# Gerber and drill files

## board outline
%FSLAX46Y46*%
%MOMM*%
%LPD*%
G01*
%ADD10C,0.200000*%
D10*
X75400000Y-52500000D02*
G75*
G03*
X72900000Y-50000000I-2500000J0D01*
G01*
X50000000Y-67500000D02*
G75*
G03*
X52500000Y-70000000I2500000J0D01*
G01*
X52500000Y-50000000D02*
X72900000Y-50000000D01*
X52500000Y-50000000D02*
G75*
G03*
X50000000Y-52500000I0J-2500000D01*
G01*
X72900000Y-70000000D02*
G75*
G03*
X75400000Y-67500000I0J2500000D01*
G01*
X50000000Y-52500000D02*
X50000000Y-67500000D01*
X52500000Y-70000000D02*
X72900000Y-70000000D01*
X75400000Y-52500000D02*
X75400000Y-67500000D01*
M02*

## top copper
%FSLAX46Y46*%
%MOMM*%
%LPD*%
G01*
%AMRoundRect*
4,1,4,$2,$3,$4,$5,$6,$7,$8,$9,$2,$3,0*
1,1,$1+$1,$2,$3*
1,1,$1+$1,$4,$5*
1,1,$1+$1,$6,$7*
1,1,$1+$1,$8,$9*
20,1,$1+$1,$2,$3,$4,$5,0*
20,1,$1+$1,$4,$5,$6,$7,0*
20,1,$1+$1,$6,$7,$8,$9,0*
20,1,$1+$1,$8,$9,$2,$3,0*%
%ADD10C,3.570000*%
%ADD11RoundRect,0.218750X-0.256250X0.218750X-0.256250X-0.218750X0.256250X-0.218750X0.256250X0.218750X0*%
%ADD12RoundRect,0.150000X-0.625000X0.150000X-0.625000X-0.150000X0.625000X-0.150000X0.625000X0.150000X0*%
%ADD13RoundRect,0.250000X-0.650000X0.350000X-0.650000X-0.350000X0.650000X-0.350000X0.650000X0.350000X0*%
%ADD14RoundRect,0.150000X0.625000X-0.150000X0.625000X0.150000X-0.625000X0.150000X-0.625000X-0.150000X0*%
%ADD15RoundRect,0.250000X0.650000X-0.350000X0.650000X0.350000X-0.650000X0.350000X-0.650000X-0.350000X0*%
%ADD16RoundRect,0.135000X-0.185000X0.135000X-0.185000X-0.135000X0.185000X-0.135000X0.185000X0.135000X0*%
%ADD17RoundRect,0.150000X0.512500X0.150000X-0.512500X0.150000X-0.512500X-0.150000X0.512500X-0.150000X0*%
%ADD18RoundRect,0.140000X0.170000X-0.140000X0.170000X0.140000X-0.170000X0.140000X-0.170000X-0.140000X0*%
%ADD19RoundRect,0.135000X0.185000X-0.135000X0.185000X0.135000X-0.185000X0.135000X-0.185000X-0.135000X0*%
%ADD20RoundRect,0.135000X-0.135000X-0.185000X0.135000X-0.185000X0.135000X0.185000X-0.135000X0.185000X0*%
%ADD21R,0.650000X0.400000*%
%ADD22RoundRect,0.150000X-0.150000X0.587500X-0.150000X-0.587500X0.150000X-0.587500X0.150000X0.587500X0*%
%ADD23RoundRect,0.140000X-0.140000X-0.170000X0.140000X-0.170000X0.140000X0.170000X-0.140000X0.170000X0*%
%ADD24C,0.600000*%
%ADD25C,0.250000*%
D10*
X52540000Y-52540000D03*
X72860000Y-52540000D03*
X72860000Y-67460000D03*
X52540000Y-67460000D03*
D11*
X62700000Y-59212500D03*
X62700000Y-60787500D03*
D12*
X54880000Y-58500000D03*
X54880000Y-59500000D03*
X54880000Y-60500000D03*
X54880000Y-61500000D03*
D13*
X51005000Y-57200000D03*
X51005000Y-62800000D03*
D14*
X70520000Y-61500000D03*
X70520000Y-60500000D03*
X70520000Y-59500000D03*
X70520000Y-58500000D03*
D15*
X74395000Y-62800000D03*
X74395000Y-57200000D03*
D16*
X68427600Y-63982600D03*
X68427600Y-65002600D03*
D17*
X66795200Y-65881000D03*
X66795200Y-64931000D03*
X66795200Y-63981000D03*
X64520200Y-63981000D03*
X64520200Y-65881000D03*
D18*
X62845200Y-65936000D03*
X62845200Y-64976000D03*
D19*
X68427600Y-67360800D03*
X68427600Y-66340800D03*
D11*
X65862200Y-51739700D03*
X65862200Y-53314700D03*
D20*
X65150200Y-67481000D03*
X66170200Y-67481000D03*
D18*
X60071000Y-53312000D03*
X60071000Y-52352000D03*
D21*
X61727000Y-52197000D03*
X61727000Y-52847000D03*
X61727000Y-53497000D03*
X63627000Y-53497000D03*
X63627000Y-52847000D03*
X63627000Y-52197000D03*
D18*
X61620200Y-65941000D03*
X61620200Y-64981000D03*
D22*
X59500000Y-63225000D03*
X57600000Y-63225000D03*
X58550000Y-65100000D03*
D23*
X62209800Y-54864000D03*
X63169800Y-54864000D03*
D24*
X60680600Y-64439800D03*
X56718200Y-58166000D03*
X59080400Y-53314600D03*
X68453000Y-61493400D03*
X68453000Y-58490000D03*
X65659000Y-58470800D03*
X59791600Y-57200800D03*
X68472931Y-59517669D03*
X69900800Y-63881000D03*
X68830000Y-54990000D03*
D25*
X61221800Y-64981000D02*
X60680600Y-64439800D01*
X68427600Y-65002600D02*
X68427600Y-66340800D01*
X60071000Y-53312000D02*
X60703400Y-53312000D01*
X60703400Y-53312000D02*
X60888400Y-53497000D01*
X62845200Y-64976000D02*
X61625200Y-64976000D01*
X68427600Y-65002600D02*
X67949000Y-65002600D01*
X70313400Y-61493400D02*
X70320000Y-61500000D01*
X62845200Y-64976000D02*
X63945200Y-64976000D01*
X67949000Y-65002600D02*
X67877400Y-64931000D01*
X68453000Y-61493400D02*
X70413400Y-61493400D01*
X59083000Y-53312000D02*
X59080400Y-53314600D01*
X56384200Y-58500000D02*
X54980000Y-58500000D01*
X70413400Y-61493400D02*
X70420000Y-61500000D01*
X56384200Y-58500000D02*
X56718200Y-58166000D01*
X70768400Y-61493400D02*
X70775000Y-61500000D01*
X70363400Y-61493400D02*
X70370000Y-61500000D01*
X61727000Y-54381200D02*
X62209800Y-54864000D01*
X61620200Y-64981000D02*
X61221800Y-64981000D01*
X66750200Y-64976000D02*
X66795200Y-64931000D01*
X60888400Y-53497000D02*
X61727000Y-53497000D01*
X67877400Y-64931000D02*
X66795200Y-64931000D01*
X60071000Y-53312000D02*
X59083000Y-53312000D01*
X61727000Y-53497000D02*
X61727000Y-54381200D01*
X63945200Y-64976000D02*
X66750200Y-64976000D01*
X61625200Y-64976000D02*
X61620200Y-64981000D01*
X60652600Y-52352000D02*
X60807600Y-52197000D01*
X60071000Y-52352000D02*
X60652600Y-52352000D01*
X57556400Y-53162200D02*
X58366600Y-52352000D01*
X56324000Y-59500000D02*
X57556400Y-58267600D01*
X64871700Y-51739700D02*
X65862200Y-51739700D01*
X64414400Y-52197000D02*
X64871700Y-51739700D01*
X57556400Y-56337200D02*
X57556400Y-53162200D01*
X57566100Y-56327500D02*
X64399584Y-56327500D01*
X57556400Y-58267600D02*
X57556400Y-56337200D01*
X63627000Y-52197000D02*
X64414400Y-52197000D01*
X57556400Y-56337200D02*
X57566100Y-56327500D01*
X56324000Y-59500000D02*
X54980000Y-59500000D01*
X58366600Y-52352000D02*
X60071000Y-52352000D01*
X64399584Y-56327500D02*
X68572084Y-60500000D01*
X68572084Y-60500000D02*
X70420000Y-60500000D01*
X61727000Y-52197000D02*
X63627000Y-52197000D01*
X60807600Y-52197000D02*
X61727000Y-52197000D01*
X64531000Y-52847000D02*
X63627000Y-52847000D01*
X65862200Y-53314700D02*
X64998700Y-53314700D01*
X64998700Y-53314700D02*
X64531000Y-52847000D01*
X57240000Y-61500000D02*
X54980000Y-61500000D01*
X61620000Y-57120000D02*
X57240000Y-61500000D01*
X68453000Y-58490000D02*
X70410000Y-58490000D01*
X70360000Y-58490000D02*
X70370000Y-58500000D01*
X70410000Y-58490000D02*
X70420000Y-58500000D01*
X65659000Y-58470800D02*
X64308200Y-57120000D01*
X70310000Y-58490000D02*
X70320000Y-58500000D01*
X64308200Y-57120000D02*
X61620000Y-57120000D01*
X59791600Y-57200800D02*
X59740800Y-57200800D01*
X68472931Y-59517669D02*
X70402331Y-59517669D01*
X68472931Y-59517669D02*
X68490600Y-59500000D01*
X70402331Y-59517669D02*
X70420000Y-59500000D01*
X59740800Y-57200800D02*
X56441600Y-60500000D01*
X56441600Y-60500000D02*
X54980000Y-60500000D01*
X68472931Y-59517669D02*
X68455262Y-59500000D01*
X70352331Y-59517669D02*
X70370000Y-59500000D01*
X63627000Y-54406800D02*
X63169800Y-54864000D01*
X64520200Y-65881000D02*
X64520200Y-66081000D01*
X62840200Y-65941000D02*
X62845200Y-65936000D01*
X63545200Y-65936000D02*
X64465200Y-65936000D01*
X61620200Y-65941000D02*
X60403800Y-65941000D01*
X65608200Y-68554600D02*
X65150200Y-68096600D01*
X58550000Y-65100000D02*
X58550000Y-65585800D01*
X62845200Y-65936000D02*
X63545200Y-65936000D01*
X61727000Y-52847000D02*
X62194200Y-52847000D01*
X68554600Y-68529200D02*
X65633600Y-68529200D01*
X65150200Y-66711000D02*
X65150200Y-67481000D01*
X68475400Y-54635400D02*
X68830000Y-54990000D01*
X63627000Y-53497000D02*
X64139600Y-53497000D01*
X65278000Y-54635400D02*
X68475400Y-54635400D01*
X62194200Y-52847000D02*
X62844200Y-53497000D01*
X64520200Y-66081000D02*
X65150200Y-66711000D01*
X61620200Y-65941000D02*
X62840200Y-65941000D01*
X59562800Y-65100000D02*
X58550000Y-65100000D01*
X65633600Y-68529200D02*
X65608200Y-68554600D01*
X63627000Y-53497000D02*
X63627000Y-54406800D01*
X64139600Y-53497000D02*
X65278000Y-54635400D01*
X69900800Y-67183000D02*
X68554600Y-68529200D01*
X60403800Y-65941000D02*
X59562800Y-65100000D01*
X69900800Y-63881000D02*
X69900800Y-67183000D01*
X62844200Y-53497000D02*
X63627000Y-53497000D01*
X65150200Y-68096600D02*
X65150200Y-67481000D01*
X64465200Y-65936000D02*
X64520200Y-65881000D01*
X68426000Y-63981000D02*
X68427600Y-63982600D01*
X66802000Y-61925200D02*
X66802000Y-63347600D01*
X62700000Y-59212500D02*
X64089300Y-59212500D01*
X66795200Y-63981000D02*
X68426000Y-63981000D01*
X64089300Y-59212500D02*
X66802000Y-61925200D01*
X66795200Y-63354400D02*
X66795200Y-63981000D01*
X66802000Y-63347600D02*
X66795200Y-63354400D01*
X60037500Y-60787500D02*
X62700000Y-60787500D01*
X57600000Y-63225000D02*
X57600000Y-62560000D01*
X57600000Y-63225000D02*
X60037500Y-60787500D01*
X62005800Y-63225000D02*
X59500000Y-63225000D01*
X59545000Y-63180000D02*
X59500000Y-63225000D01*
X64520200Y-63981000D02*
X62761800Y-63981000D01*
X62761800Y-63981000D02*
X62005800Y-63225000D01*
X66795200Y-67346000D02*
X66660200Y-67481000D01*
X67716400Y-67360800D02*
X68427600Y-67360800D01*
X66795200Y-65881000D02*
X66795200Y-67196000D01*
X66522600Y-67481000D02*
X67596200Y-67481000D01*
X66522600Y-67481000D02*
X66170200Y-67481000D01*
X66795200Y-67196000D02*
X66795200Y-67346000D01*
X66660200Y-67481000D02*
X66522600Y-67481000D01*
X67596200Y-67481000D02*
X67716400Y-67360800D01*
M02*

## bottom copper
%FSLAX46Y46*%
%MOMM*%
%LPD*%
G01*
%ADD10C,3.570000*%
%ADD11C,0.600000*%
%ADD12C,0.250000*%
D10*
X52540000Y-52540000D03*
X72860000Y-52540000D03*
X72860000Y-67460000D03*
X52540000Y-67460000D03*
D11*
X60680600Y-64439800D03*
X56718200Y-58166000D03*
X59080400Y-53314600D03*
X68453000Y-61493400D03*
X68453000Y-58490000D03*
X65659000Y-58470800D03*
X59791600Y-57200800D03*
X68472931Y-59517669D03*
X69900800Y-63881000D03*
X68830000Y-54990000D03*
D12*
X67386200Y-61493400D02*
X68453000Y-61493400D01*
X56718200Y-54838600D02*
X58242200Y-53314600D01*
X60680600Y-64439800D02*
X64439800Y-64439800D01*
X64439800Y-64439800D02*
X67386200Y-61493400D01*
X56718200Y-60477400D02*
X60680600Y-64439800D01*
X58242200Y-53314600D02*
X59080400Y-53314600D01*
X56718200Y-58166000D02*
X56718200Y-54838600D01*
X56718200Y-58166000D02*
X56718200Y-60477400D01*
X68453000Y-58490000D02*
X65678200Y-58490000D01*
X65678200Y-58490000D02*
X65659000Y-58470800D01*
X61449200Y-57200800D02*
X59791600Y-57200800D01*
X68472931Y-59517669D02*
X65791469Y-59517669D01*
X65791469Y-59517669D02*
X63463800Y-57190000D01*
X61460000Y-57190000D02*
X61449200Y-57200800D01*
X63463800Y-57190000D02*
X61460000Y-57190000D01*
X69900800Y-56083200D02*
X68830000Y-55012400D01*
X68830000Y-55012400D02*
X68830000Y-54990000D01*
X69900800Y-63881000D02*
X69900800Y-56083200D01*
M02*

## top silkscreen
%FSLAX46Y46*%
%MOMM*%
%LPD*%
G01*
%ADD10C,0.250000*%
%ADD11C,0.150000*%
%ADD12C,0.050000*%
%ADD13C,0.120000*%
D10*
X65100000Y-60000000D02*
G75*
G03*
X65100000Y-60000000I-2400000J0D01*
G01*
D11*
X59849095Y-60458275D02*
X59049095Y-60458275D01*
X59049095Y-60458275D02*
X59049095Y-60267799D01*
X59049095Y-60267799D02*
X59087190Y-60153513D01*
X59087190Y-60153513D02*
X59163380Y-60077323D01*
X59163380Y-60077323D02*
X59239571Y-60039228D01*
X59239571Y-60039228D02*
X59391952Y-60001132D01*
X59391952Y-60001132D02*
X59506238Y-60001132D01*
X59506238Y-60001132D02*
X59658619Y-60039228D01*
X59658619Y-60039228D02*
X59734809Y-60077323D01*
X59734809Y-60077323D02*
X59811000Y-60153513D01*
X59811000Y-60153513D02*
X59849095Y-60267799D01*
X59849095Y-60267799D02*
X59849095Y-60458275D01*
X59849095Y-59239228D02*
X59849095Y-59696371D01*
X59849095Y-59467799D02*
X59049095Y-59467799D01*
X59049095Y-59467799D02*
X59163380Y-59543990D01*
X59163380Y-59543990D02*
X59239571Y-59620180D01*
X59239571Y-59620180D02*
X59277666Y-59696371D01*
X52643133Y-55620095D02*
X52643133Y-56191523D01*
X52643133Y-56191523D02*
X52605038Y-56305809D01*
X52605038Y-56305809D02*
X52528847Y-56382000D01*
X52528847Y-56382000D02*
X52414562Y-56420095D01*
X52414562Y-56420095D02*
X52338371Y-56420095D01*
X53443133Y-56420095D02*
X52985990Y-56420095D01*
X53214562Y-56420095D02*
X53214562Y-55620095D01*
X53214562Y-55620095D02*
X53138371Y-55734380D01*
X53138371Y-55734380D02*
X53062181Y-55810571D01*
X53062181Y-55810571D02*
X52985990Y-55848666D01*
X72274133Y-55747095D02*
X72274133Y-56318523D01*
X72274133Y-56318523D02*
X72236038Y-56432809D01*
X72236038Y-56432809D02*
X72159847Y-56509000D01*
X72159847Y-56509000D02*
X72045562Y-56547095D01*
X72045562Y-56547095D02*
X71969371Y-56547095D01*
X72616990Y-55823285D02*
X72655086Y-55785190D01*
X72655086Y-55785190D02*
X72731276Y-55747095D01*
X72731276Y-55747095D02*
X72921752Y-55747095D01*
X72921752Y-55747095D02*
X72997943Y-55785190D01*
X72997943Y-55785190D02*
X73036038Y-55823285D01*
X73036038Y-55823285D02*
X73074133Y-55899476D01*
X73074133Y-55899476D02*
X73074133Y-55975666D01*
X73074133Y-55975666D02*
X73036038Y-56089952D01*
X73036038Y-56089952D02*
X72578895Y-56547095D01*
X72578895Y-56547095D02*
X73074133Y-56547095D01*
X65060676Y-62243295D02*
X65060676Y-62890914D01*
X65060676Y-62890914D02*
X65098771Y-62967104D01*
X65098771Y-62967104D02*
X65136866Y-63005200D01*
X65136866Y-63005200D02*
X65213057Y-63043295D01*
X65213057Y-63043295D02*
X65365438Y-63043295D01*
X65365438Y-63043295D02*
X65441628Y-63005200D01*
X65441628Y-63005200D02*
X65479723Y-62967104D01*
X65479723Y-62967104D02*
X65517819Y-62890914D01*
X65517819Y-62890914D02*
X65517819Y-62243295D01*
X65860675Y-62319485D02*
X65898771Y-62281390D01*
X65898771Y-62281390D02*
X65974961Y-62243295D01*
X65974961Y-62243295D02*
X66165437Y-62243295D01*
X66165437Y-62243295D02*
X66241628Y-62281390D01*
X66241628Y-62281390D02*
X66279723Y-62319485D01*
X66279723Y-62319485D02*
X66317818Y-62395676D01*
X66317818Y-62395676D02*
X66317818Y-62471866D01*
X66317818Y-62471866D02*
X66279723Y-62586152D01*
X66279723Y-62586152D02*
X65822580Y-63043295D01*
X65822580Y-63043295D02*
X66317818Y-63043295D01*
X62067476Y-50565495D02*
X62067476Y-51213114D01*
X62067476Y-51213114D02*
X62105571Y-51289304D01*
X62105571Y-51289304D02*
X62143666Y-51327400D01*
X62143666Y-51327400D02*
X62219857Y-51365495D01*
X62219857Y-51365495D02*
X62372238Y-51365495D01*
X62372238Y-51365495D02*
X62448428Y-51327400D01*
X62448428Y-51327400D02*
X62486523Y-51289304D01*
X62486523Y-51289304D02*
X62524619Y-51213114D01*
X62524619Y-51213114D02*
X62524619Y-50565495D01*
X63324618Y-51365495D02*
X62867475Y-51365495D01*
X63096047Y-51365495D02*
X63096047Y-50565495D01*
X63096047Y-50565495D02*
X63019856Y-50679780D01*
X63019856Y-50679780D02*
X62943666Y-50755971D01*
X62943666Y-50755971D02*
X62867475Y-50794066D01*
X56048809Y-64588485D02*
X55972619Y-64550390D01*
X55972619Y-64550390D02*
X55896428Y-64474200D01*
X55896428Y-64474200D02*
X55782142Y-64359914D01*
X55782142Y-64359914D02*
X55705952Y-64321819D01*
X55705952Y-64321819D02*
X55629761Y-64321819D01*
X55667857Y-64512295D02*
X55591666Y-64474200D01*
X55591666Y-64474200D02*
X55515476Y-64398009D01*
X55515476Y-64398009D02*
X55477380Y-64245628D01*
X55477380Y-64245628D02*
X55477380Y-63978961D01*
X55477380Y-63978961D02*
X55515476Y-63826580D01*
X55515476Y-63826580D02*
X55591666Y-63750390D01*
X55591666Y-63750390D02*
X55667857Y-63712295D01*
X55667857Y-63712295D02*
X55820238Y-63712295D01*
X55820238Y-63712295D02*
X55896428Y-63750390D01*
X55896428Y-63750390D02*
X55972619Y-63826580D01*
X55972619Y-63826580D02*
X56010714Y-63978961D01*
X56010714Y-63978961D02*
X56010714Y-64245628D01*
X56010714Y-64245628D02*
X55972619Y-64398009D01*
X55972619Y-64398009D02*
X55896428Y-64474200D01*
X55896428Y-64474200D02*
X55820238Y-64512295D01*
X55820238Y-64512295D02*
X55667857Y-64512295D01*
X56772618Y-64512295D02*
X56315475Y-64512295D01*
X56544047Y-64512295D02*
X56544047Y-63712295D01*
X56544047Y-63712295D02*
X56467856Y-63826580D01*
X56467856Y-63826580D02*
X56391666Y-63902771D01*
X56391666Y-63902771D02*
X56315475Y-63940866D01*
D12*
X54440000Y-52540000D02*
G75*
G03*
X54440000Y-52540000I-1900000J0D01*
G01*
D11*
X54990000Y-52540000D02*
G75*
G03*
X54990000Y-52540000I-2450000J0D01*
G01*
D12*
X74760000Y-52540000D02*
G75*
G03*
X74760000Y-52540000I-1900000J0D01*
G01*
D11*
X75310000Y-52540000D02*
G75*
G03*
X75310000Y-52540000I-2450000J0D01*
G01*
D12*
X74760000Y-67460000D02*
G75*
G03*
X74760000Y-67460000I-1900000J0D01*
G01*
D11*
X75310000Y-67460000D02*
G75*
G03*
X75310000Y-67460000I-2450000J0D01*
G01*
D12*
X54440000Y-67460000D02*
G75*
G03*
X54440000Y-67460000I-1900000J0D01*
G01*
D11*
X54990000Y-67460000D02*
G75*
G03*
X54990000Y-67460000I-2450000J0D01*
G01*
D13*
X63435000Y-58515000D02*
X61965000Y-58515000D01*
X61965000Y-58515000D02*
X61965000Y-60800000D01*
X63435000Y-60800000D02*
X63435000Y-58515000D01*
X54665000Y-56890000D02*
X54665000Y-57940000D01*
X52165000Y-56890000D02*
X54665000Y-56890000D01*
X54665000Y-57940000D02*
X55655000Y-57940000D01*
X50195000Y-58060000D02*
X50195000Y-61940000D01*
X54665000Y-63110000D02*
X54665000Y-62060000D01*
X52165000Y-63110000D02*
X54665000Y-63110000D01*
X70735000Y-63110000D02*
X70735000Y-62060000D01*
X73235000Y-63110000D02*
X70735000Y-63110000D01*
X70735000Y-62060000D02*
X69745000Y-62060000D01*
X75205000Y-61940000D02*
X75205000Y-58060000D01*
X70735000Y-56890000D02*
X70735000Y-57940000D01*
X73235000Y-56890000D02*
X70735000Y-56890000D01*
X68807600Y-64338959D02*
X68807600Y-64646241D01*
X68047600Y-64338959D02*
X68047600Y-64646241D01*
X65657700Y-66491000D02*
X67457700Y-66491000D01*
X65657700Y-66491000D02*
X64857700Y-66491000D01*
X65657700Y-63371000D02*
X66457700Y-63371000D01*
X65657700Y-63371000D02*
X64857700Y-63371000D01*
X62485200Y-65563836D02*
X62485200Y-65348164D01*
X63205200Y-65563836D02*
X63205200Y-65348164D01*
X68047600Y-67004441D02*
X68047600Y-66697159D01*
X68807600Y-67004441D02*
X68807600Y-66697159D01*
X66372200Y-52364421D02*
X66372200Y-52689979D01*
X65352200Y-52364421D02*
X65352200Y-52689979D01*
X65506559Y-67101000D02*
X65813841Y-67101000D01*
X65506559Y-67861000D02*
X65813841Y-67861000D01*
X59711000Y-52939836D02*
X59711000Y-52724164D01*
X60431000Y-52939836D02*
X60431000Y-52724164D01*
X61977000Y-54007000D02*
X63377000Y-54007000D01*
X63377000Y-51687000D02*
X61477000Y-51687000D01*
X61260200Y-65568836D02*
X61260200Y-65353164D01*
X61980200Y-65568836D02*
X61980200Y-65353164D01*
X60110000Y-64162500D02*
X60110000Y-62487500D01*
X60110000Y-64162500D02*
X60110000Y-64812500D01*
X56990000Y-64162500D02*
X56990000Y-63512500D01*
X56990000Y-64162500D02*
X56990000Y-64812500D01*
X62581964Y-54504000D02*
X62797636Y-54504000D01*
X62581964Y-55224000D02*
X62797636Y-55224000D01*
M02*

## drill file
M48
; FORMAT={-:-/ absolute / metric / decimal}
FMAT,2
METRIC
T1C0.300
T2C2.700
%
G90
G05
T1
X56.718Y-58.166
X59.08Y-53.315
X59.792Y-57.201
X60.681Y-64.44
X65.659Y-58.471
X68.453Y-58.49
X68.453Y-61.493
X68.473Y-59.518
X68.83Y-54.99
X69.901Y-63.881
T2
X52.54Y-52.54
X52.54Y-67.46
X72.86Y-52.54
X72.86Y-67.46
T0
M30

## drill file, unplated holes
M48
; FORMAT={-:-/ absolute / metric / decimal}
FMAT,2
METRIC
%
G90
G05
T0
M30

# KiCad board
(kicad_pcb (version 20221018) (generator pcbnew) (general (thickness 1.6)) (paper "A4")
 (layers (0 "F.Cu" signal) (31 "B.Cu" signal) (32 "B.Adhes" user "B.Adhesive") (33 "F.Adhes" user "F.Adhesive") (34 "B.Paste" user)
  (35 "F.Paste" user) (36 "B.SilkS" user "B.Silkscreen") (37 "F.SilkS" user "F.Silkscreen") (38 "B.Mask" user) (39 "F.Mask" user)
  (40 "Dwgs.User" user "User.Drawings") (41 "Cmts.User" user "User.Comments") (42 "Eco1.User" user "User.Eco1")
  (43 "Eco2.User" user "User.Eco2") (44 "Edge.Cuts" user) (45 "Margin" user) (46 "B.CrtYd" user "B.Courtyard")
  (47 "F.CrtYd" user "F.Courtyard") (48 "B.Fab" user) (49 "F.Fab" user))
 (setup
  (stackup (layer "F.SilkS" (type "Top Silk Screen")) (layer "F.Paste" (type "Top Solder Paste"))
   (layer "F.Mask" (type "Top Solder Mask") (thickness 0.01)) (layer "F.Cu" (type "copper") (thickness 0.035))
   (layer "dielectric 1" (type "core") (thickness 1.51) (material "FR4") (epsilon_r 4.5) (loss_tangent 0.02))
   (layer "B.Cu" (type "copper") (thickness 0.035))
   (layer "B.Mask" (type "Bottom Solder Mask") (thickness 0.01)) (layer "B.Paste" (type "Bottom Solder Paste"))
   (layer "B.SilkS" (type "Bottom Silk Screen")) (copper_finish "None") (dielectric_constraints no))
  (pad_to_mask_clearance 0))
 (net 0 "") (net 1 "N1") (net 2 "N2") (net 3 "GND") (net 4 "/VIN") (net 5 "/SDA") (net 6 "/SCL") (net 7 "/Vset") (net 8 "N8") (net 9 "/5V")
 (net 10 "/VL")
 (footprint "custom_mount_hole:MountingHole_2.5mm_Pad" (layer "F.Cu") (at 52.54 52.54)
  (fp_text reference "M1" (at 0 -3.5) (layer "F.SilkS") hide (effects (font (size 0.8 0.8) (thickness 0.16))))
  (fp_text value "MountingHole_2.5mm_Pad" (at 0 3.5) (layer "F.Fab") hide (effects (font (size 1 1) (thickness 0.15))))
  (fp_circle (center 0 0) (end 1.9 0) (stroke (width 0.05) (type solid)) (fill none) (layer "F.SilkS"))
  (fp_circle (center 0 0) (end 2.45 0) (stroke (width 0.15) (type solid)) (fill none) (layer "F.SilkS"))
  (pad "~" thru_hole circle (at 0 0) (size 3.57 3.57) (drill 2.7) (layers "*.Cu" "*.Mask")))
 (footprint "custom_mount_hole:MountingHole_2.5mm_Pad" (layer "F.Cu") (at 72.86 52.54)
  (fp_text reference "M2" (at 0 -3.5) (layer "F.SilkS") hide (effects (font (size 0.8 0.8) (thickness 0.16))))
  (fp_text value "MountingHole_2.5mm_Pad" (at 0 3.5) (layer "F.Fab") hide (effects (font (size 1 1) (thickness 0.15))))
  (fp_circle (center 0 0) (end 1.9 0) (stroke (width 0.05) (type solid)) (fill none) (layer "F.SilkS"))
  (fp_circle (center 0 0) (end 2.45 0) (stroke (width 0.15) (type solid)) (fill none) (layer "F.SilkS"))
  (pad "~" thru_hole circle (at 0 0) (size 3.57 3.57) (drill 2.7) (layers "*.Cu" "*.Mask")))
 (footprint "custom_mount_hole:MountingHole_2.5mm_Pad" (layer "F.Cu") (at 72.86 67.46)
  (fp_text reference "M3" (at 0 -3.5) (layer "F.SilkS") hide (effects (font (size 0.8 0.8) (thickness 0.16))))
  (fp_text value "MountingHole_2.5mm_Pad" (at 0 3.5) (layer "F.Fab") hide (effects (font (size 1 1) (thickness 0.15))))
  (fp_circle (center 0 0) (end 1.9 0) (stroke (width 0.05) (type solid)) (fill none) (layer "F.SilkS"))
  (fp_circle (center 0 0) (end 2.45 0) (stroke (width 0.15) (type solid)) (fill none) (layer "F.SilkS"))
  (pad "~" thru_hole circle (at 0 0) (size 3.57 3.57) (drill 2.7) (layers "*.Cu" "*.Mask")))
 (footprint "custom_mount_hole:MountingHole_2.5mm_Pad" (layer "F.Cu") (at 52.54 67.46)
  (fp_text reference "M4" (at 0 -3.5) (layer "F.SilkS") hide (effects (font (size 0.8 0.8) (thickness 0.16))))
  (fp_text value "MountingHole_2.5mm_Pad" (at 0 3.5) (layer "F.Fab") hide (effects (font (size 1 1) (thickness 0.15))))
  (fp_circle (center 0 0) (end 1.9 0) (stroke (width 0.05) (type solid)) (fill none) (layer "F.SilkS"))
  (fp_circle (center 0 0) (end 2.45 0) (stroke (width 0.15) (type solid)) (fill none) (layer "F.SilkS"))
  (pad "~" thru_hole circle (at 0 0) (size 3.57 3.57) (drill 2.7) (layers "*.Cu" "*.Mask")))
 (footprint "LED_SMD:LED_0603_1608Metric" (layer "F.Cu") (at 62.7 60 -90)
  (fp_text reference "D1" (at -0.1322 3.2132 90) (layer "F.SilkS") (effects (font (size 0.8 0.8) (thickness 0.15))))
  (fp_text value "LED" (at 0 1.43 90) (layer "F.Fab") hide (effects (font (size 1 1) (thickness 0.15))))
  (fp_line (start -1.485 -0.735) (end -1.485 0.735) (stroke (width 0.12) (type solid)) (layer "F.SilkS"))
  (fp_line (start -1.485 0.735) (end 0.8 0.735) (stroke (width 0.12) (type solid)) (layer "F.SilkS"))
  (fp_line (start 0.8 -0.735) (end -1.485 -0.735) (stroke (width 0.12) (type solid)) (layer "F.SilkS"))
  (pad "1" smd roundrect (at -0.7875 0 270) (size 0.875 0.95) (layers "F.Cu" "F.Paste" "F.Mask") (roundrect_rratio 0.25) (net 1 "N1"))
  (pad "2" smd roundrect (at 0.7875 0 270) (size 0.875 0.95) (layers "F.Cu" "F.Paste" "F.Mask") (roundrect_rratio 0.25) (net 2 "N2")))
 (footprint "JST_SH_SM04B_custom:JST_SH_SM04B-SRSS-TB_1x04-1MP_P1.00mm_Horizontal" (layer "F.Cu") (at 52.88 60 -90)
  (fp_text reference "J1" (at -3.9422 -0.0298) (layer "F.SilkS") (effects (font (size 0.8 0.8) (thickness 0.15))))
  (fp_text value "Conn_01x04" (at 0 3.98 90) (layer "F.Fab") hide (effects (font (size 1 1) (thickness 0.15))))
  (fp_line (start -3.11 -1.785) (end -2.06 -1.785) (stroke (width 0.12) (type solid)) (layer "F.SilkS"))
  (fp_line (start -3.11 0.715) (end -3.11 -1.785) (stroke (width 0.12) (type solid)) (layer "F.SilkS"))
  (fp_line (start -2.06 -1.785) (end -2.06 -2.775) (stroke (width 0.12) (type solid)) (layer "F.SilkS"))
  (fp_line (start -1.94 2.685) (end 1.94 2.685) (stroke (width 0.12) (type solid)) (layer "F.SilkS"))
  (fp_line (start 3.11 -1.785) (end 2.06 -1.785) (stroke (width 0.12) (type solid)) (layer "F.SilkS"))
  (fp_line (start 3.11 0.715) (end 3.11 -1.785) (stroke (width 0.12) (type solid)) (layer "F.SilkS"))
  (pad "1" smd roundrect (at -1.5 -2 270) (size 0.6 1.55) (layers "F.Cu" "F.Paste" "F.Mask") (roundrect_rratio 0.25) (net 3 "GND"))
  (pad "2" smd roundrect (at -0.5 -2 270) (size 0.6 1.55) (layers "F.Cu" "F.Paste" "F.Mask") (roundrect_rratio 0.25) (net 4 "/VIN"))
  (pad "3" smd roundrect (at 0.5 -2 270) (size 0.6 1.55) (layers "F.Cu" "F.Paste" "F.Mask") (roundrect_rratio 0.25) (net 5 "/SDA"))
  (pad "4" smd roundrect (at 1.5 -2 270) (size 0.6 1.55) (layers "F.Cu" "F.Paste" "F.Mask") (roundrect_rratio 0.25) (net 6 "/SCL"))
  (pad "MP" smd roundrect (at -2.8 1.875 270) (size 1.2 1.8) (layers "F.Cu" "F.Paste" "F.Mask") (roundrect_rratio 0.2083333333))
  (pad "MP" smd roundrect (at 2.8 1.875 270) (size 1.2 1.8) (layers "F.Cu" "F.Paste" "F.Mask") (roundrect_rratio 0.2083333333)))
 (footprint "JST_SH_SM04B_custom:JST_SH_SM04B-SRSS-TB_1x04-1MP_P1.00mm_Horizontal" (layer "F.Cu") (at 72.52 60 90)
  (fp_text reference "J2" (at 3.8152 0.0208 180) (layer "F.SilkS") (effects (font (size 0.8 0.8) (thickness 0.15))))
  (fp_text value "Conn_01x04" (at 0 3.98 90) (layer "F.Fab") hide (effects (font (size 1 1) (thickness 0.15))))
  (fp_line (start -3.11 -1.785) (end -2.06 -1.785) (stroke (width 0.12) (type solid)) (layer "F.SilkS"))
  (fp_line (start -3.11 0.715) (end -3.11 -1.785) (stroke (width 0.12) (type solid)) (layer "F.SilkS"))
  (fp_line (start -2.06 -1.785) (end -2.06 -2.775) (stroke (width 0.12) (type solid)) (layer "F.SilkS"))
  (fp_line (start -1.94 2.685) (end 1.94 2.685) (stroke (width 0.12) (type solid)) (layer "F.SilkS"))
  (fp_line (start 3.11 -1.785) (end 2.06 -1.785) (stroke (width 0.12) (type solid)) (layer "F.SilkS"))
  (fp_line (start 3.11 0.715) (end 3.11 -1.785) (stroke (width 0.12) (type solid)) (layer "F.SilkS"))
  (pad "1" smd roundrect (at -1.5 -2 90) (size 0.6 1.55) (layers "F.Cu" "F.Paste" "F.Mask") (roundrect_rratio 0.25) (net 3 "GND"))
  (pad "2" smd roundrect (at -0.5 -2 90) (size 0.6 1.55) (layers "F.Cu" "F.Paste" "F.Mask") (roundrect_rratio 0.25) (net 4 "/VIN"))
  (pad "3" smd roundrect (at 0.5 -2 90) (size 0.6 1.55) (layers "F.Cu" "F.Paste" "F.Mask") (roundrect_rratio 0.25) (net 5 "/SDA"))
  (pad "4" smd roundrect (at 1.5 -2 90) (size 0.6 1.55) (layers "F.Cu" "F.Paste" "F.Mask") (roundrect_rratio 0.25) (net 6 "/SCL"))
  (pad "MP" smd roundrect (at -2.8 1.875 90) (size 1.2 1.8) (layers "F.Cu" "F.Paste" "F.Mask") (roundrect_rratio 0.2083333333))
  (pad "MP" smd roundrect (at 2.8 1.875 90) (size 1.2 1.8) (layers "F.Cu" "F.Paste" "F.Mask") (roundrect_rratio 0.2083333333)))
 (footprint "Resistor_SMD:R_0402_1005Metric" (layer "F.Cu") (at 68.4276 64.4926 -90)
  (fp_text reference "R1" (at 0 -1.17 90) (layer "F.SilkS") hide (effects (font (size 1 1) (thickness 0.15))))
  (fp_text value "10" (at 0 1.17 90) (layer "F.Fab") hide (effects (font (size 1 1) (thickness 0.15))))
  (fp_line (start -0.153641 -0.38) (end 0.153641 -0.38) (stroke (width 0.12) (type solid)) (layer "F.SilkS"))
  (fp_line (start -0.153641 0.38) (end 0.153641 0.38) (stroke (width 0.12) (type solid)) (layer "F.SilkS"))
  (pad "1" smd roundrect (at -0.51 0 270) (size 0.54 0.64) (layers "F.Cu" "F.Paste" "F.Mask") (roundrect_rratio 0.25) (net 1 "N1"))
  (pad "2" smd roundrect (at 0.51 0 270) (size 0.54 0.64) (layers "F.Cu" "F.Paste" "F.Mask") (roundrect_rratio 0.25) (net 3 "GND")))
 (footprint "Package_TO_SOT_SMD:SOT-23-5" (layer "F.Cu") (at 65.6577 64.931 180)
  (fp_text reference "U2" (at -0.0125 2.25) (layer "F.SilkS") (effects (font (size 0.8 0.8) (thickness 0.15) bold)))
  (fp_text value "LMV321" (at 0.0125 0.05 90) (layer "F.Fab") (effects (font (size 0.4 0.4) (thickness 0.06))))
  (fp_line (start 0 -1.56) (end -1.8 -1.56) (stroke (width 0.12) (type solid)) (layer "F.SilkS"))
  (fp_line (start 0 -1.56) (end 0.8 -1.56) (stroke (width 0.12) (type solid)) (layer "F.SilkS"))
  (fp_line (start 0 1.56) (end -0.8 1.56) (stroke (width 0.12) (type solid)) (layer "F.SilkS"))
  (fp_line (start 0 1.56) (end 0.8 1.56) (stroke (width 0.12) (type solid)) (layer "F.SilkS"))
  (pad "1" smd roundrect (at -1.1375 -0.95 180) (size 1.325 0.6) (layers "F.Cu" "F.Paste" "F.Mask") (roundrect_rratio 0.25) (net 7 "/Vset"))
  (pad "2" smd roundrect (at -1.1375 0 180) (size 1.325 0.6) (layers "F.Cu" "F.Paste" "F.Mask") (roundrect_rratio 0.25) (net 3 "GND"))
  (pad "3" smd roundrect (at -1.1375 0.95 180) (size 1.325 0.6) (layers "F.Cu" "F.Paste" "F.Mask") (roundrect_rratio 0.25) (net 1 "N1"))
  (pad "4" smd roundrect (at 1.1375 0.95 180) (size 1.325 0.6) (layers "F.Cu" "F.Paste" "F.Mask") (roundrect_rratio 0.25) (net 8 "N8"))
  (pad "5" smd roundrect (at 1.1375 -0.95 180) (size 1.325 0.6) (layers "F.Cu" "F.Paste" "F.Mask") (roundrect_rratio 0.25) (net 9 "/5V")))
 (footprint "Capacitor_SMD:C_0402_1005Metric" (layer "F.Cu") (at 62.8452 65.456 90)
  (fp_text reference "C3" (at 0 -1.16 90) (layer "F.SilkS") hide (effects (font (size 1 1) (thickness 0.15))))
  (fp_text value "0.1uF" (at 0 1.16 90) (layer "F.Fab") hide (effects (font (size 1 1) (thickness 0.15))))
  (fp_line (start -0.107836 -0.36) (end 0.107836 -0.36) (stroke (width 0.12) (type solid)) (layer "F.SilkS"))
  (fp_line (start -0.107836 0.36) (end 0.107836 0.36) (stroke (width 0.12) (type solid)) (layer "F.SilkS"))
  (pad "1" smd roundrect (at -0.48 0 90) (size 0.56 0.62) (layers "F.Cu" "F.Paste" "F.Mask") (roundrect_rratio 0.25) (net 9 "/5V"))
  (pad "2" smd roundrect (at 0.48 0 90) (size 0.56 0.62) (layers "F.Cu" "F.Paste" "F.Mask") (roundrect_rratio 0.25) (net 3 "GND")))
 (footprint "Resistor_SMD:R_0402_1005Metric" (layer "F.Cu") (at 68.4276 66.8508 90)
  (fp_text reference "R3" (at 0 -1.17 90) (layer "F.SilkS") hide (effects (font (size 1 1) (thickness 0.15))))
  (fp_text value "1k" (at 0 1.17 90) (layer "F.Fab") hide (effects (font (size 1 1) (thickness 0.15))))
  (fp_line (start -0.153641 -0.38) (end 0.153641 -0.38) (stroke (width 0.12) (type solid)) (layer "F.SilkS"))
  (fp_line (start -0.153641 0.38) (end 0.153641 0.38) (stroke (width 0.12) (type solid)) (layer "F.SilkS"))
  (pad "1" smd roundrect (at -0.51 0 90) (size 0.54 0.64) (layers "F.Cu" "F.Paste" "F.Mask") (roundrect_rratio 0.25) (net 7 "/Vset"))
  (pad "2" smd roundrect (at 0.51 0 90) (size 0.54 0.64) (layers "F.Cu" "F.Paste" "F.Mask") (roundrect_rratio 0.25) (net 3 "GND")))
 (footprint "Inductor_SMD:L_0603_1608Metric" (layer "F.Cu") (at 65.8622 52.5272 -90)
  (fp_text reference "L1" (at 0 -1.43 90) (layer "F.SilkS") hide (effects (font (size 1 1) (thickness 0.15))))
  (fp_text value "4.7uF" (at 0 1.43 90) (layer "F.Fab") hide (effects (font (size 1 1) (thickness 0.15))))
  (fp_line (start -0.162779 -0.51) (end 0.162779 -0.51) (stroke (width 0.12) (type solid)) (layer "F.SilkS"))
  (fp_line (start -0.162779 0.51) (end 0.162779 0.51) (stroke (width 0.12) (type solid)) (layer "F.SilkS"))
  (pad "1" smd roundrect (at -0.7875 0 270) (size 0.875 0.95) (layers "F.Cu" "F.Paste" "F.Mask") (roundrect_rratio 0.25) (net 4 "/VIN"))
  (pad "2" smd roundrect (at 0.7875 0 270) (size 0.875 0.95) (layers "F.Cu" "F.Paste" "F.Mask") (roundrect_rratio 0.25) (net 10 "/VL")))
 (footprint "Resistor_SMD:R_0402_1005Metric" (layer "F.Cu") (at 65.6602 67.481)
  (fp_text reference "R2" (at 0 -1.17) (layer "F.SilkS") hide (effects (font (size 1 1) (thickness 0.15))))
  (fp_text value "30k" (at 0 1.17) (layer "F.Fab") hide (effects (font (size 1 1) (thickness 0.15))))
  (fp_line (start -0.153641 -0.38) (end 0.153641 -0.38) (stroke (width 0.12) (type solid)) (layer "F.SilkS"))
  (fp_line (start -0.153641 0.38) (end 0.153641 0.38) (stroke (width 0.12) (type solid)) (layer "F.SilkS"))
  (pad "1" smd roundrect (at -0.51 0) (size 0.54 0.64) (layers "F.Cu" "F.Paste" "F.Mask") (roundrect_rratio 0.25) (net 9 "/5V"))
  (pad "2" smd roundrect (at 0.51 0) (size 0.54 0.64) (layers "F.Cu" "F.Paste" "F.Mask") (roundrect_rratio 0.25) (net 7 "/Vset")))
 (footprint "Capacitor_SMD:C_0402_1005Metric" (layer "F.Cu") (at 60.071 52.832 90)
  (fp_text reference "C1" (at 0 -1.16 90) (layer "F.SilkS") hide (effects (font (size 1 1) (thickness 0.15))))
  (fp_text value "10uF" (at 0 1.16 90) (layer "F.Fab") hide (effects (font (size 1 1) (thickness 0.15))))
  (fp_line (start -0.107836 -0.36) (end 0.107836 -0.36) (stroke (width 0.12) (type solid)) (layer "F.SilkS"))
  (fp_line (start -0.107836 0.36) (end 0.107836 0.36) (stroke (width 0.12) (type solid)) (layer "F.SilkS"))
  (pad "1" smd roundrect (at -0.48 0 90) (size 0.56 0.62) (layers "F.Cu" "F.Paste" "F.Mask") (roundrect_rratio 0.25) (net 3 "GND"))
  (pad "2" smd roundrect (at 0.48 0 90) (size 0.56 0.62) (layers "F.Cu" "F.Paste" "F.Mask") (roundrect_rratio 0.25) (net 4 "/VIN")))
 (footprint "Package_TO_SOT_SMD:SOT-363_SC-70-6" (layer "F.Cu") (at 62.677 52.847)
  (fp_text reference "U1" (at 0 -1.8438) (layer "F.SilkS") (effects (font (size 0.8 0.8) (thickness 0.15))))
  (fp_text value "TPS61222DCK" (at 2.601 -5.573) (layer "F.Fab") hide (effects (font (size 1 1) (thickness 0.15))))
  (fp_line (start -0.7 1.16) (end 0.7 1.16) (stroke (width 0.12) (type solid)) (layer "F.SilkS"))
  (fp_line (start 0.7 -1.16) (end -1.2 -1.16) (stroke (width 0.12) (type solid)) (layer "F.SilkS"))
  (pad "1" smd rect (at -0.95 -0.65) (size 0.65 0.4) (layers "F.Cu" "F.Paste" "F.Mask") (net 4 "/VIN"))
  (pad "2" smd rect (at -0.95 0) (size 0.65 0.4) (layers "F.Cu" "F.Paste" "F.Mask") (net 9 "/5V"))
  (pad "3" smd rect (at -0.95 0.65) (size 0.65 0.4) (layers "F.Cu" "F.Paste" "F.Mask") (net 3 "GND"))
  (pad "4" smd rect (at 0.95 0.65) (size 0.65 0.4) (layers "F.Cu" "F.Paste" "F.Mask") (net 9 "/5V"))
  (pad "5" smd rect (at 0.95 0) (size 0.65 0.4) (layers "F.Cu" "F.Paste" "F.Mask") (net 10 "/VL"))
  (pad "6" smd rect (at 0.95 -0.65) (size 0.65 0.4) (layers "F.Cu" "F.Paste" "F.Mask") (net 4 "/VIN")))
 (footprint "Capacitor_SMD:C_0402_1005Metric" (layer "F.Cu") (at 61.6202 65.461 90)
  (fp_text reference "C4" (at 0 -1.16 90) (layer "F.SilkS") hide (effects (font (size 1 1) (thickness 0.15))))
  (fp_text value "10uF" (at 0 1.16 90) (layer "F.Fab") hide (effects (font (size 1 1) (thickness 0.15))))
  (fp_line (start -0.107836 -0.36) (end 0.107836 -0.36) (stroke (width 0.12) (type solid)) (layer "F.SilkS"))
  (fp_line (start -0.107836 0.36) (end 0.107836 0.36) (stroke (width 0.12) (type solid)) (layer "F.SilkS"))
  (pad "1" smd roundrect (at -0.48 0 90) (size 0.56 0.62) (layers "F.Cu" "F.Paste" "F.Mask") (roundrect_rratio 0.25) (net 9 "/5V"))
  (pad "2" smd roundrect (at 0.48 0 90) (size 0.56 0.62) (layers "F.Cu" "F.Paste" "F.Mask") (roundrect_rratio 0.25) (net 3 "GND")))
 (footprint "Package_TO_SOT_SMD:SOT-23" (layer "F.Cu") (at 58.55 64.1625 -90)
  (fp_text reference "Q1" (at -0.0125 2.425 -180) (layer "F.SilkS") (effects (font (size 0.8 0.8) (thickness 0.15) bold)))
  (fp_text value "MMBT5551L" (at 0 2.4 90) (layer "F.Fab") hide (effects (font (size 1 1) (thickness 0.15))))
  (fp_line (start 0 -1.56) (end -1.675 -1.56) (stroke (width 0.12) (type solid)) (layer "F.SilkS"))
  (fp_line (start 0 -1.56) (end 0.65 -1.56) (stroke (width 0.12) (type solid)) (layer "F.SilkS"))
  (fp_line (start 0 1.56) (end -0.65 1.56) (stroke (width 0.12) (type solid)) (layer "F.SilkS"))
  (fp_line (start 0 1.56) (end 0.65 1.56) (stroke (width 0.12) (type solid)) (layer "F.SilkS"))
  (pad "1" smd roundrect (at -0.9375 -0.95 270) (size 1.475 0.6) (layers "F.Cu" "F.Paste" "F.Mask") (roundrect_rratio 0.25) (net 8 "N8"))
  (pad "2" smd roundrect (at -0.9375 0.95 270) (size 1.475 0.6) (layers "F.Cu" "F.Paste" "F.Mask") (roundrect_rratio 0.25) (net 2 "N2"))
  (pad "3" smd roundrect (at 0.9375 0 270) (size 1.475 0.6) (layers "F.Cu" "F.Paste" "F.Mask") (roundrect_rratio 0.25) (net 9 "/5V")))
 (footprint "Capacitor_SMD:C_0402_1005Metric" (layer "F.Cu") (at 62.6898 54.864)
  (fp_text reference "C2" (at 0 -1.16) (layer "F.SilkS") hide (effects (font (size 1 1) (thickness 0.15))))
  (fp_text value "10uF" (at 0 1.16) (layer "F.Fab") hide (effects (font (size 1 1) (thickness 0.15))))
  (fp_line (start -0.107836 -0.36) (end 0.107836 -0.36) (stroke (width 0.12) (type solid)) (layer "F.SilkS"))
  (fp_line (start -0.107836 0.36) (end 0.107836 0.36) (stroke (width 0.12) (type solid)) (layer "F.SilkS"))
  (pad "1" smd roundrect (at -0.48 0) (size 0.56 0.62) (layers "F.Cu" "F.Paste" "F.Mask") (roundrect_rratio 0.25) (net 3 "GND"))
  (pad "2" smd roundrect (at 0.48 0) (size 0.56 0.62) (layers "F.Cu" "F.Paste" "F.Mask") (roundrect_rratio 0.25) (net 9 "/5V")))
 (gr_circle (center 62.7 60) (end 65.1 60) (stroke (width 0.25) (type solid)) (fill none) (layer "F.SilkS"))
 (gr_arc (start 72.9 50) (mid 74.667767 50.732233) (end 75.4 52.5) (stroke (width 0.2) (type solid)) (layer "Edge.Cuts"))
 (gr_arc (start 52.5 70) (mid 50.732233 69.267767) (end 50 67.5) (stroke (width 0.2) (type solid)) (layer "Edge.Cuts"))
 (gr_line (start 52.5 50) (end 72.9 50) (stroke (width 0.2) (type solid)) (layer "Edge.Cuts"))
 (gr_arc (start 50 52.5) (mid 50.732233 50.732233) (end 52.5 50) (stroke (width 0.2) (type solid)) (layer "Edge.Cuts"))
 (gr_arc (start 75.4 67.5) (mid 74.667767 69.267767) (end 72.9 70) (stroke (width 0.2) (type solid)) (layer "Edge.Cuts"))
 (gr_line (start 50 52.5) (end 50 67.5) (stroke (width 0.2) (type solid)) (layer "Edge.Cuts"))
 (gr_line (start 52.5 70) (end 72.9 70) (stroke (width 0.2) (type solid)) (layer "Edge.Cuts"))
 (gr_line (start 75.4 52.5) (end 75.4 67.5) (stroke (width 0.2) (type solid)) (layer "Edge.Cuts"))
 (segment (start 61.2218 64.981) (end 60.6806 64.4398) (width 0.25) (layer "F.Cu") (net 3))
 (segment (start 68.4276 65.0026) (end 68.4276 66.3408) (width 0.25) (layer "F.Cu") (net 3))
 (segment (start 60.071 53.312) (end 60.7034 53.312) (width 0.25) (layer "F.Cu") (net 3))
 (segment (start 60.7034 53.312) (end 60.8884 53.497) (width 0.25) (layer "F.Cu") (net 3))
 (segment (start 62.8452 64.976) (end 61.6252 64.976) (width 0.25) (layer "F.Cu") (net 3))
 (segment (start 68.4276 65.0026) (end 67.949 65.0026) (width 0.25) (layer "F.Cu") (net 3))
 (segment (start 70.3134 61.4934) (end 70.32 61.5) (width 0.25) (layer "F.Cu") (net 3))
 (segment (start 62.8452 64.976) (end 63.9452 64.976) (width 0.25) (layer "F.Cu") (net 3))
 (segment (start 67.949 65.0026) (end 67.8774 64.931) (width 0.25) (layer "F.Cu") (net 3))
 (segment (start 68.453 61.4934) (end 70.4134 61.4934) (width 0.25) (layer "F.Cu") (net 3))
 (segment (start 59.083 53.312) (end 59.0804 53.3146) (width 0.25) (layer "F.Cu") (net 3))
 (segment (start 56.3842 58.5) (end 54.98 58.5) (width 0.25) (layer "F.Cu") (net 3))
 (segment (start 70.4134 61.4934) (end 70.42 61.5) (width 0.25) (layer "F.Cu") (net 3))
 (segment (start 56.3842 58.5) (end 56.7182 58.166) (width 0.25) (layer "F.Cu") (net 3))
 (segment (start 70.7684 61.4934) (end 70.775 61.5) (width 0.25) (layer "F.Cu") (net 3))
 (segment (start 70.3634 61.4934) (end 70.37 61.5) (width 0.25) (layer "F.Cu") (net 3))
 (segment (start 61.727 54.3812) (end 62.2098 54.864) (width 0.25) (layer "F.Cu") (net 3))
 (segment (start 61.6202 64.981) (end 61.2218 64.981) (width 0.25) (layer "F.Cu") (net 3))
 (segment (start 66.7502 64.976) (end 66.7952 64.931) (width 0.25) (layer "F.Cu") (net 3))
 (segment (start 60.8884 53.497) (end 61.727 53.497) (width 0.25) (layer "F.Cu") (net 3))
 (segment (start 67.8774 64.931) (end 66.7952 64.931) (width 0.25) (layer "F.Cu") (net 3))
 (segment (start 60.071 53.312) (end 59.083 53.312) (width 0.25) (layer "F.Cu") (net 3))
 (segment (start 61.727 53.497) (end 61.727 54.3812) (width 0.25) (layer "F.Cu") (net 3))
 (segment (start 63.9452 64.976) (end 66.7502 64.976) (width 0.25) (layer "F.Cu") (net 3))
 (segment (start 61.6252 64.976) (end 61.6202 64.981) (width 0.25) (layer "F.Cu") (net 3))
 (via (at 60.6806 64.4398) (size 0.6) (drill 0.3) (layers "F.Cu" "B.Cu") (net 3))
 (via (at 56.7182 58.166) (size 0.6) (drill 0.3) (layers "F.Cu" "B.Cu") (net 3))
 (via (at 59.0804 53.3146) (size 0.6) (drill 0.3) (layers "F.Cu" "B.Cu") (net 3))
 (via (at 68.453 61.4934) (size 0.6) (drill 0.3) (layers "F.Cu" "B.Cu") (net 3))
 (segment (start 67.3862 61.4934) (end 68.453 61.4934) (width 0.25) (layer "B.Cu") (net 3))
 (segment (start 56.7182 54.8386) (end 58.2422 53.3146) (width 0.25) (layer "B.Cu") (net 3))
 (segment (start 60.6806 64.4398) (end 64.4398 64.4398) (width 0.25) (layer "B.Cu") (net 3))
 (segment (start 64.4398 64.4398) (end 67.3862 61.4934) (width 0.25) (layer "B.Cu") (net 3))
 (segment (start 56.7182 60.4774) (end 60.6806 64.4398) (width 0.25) (layer "B.Cu") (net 3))
 (segment (start 58.2422 53.3146) (end 59.0804 53.3146) (width 0.25) (layer "B.Cu") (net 3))
 (segment (start 56.7182 58.166) (end 56.7182 54.8386) (width 0.25) (layer "B.Cu") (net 3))
 (segment (start 56.7182 58.166) (end 56.7182 60.4774) (width 0.25) (layer "B.Cu") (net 3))
 (segment (start 60.6526 52.352) (end 60.8076 52.197) (width 0.25) (layer "F.Cu") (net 4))
 (segment (start 60.071 52.352) (end 60.6526 52.352) (width 0.25) (layer "F.Cu") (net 4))
 (segment (start 57.5564 53.1622) (end 58.3666 52.352) (width 0.25) (layer "F.Cu") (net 4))
 (segment (start 56.324 59.5) (end 57.5564 58.2676) (width 0.25) (layer "F.Cu") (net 4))
 (segment (start 64.8717 51.7397) (end 65.8622 51.7397) (width 0.25) (layer "F.Cu") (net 4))
 (segment (start 64.4144 52.197) (end 64.8717 51.7397) (width 0.25) (layer "F.Cu") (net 4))
 (segment (start 57.5564 56.3372) (end 57.5564 53.1622) (width 0.25) (layer "F.Cu") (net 4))
 (segment (start 57.5661 56.3275) (end 64.399584 56.3275) (width 0.25) (layer "F.Cu") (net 4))
 (segment (start 57.5564 58.2676) (end 57.5564 56.3372) (width 0.25) (layer "F.Cu") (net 4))
 (segment (start 63.627 52.197) (end 64.4144 52.197) (width 0.25) (layer "F.Cu") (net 4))
 (segment (start 57.5564 56.3372) (end 57.5661 56.3275) (width 0.25) (layer "F.Cu") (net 4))
 (segment (start 56.324 59.5) (end 54.98 59.5) (width 0.25) (layer "F.Cu") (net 4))
 (segment (start 58.3666 52.352) (end 60.071 52.352) (width 0.25) (layer "F.Cu") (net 4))
 (segment (start 64.399584 56.3275) (end 68.572084 60.5) (width 0.25) (layer "F.Cu") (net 4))
 (segment (start 68.572084 60.5) (end 70.42 60.5) (width 0.25) (layer "F.Cu") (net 4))
 (segment (start 61.727 52.197) (end 63.627 52.197) (width 0.25) (layer "F.Cu") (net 4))
 (segment (start 60.8076 52.197) (end 61.727 52.197) (width 0.25) (layer "F.Cu") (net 4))
 (segment (start 64.531 52.847) (end 63.627 52.847) (width 0.25) (layer "F.Cu") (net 10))
 (segment (start 65.8622 53.3147) (end 64.9987 53.3147) (width 0.25) (layer "F.Cu") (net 10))
 (segment (start 64.9987 53.3147) (end 64.531 52.847) (width 0.25) (layer "F.Cu") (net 10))
 (segment (start 57.24 61.5) (end 54.98 61.5) (width 0.25) (layer "F.Cu") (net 6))
 (segment (start 61.62 57.12) (end 57.24 61.5) (width 0.25) (layer "F.Cu") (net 6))
 (segment (start 68.453 58.49) (end 70.41 58.49) (width 0.25) (layer "F.Cu") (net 6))
 (segment (start 70.36 58.49) (end 70.37 58.5) (width 0.25) (layer "F.Cu") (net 6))
 (segment (start 70.41 58.49) (end 70.42 58.5) (width 0.25) (layer "F.Cu") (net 6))
 (segment (start 65.659 58.4708) (end 64.3082 57.12) (width 0.25) (layer "F.Cu") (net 6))
 (segment (start 70.31 58.49) (end 70.32 58.5) (width 0.25) (layer "F.Cu") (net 6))
 (segment (start 64.3082 57.12) (end 61.62 57.12) (width 0.25) (layer "F.Cu") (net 6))
 (via (at 68.453 58.49) (size 0.6) (drill 0.3) (layers "F.Cu" "B.Cu") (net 6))
 (via (at 65.659 58.4708) (size 0.6) (drill 0.3) (layers "F.Cu" "B.Cu") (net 6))
 (segment (start 68.453 58.49) (end 65.6782 58.49) (width 0.25) (layer "B.Cu") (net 6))
 (segment (start 65.6782 58.49) (end 65.659 58.4708) (width 0.25) (layer "B.Cu") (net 6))
 (segment (start 59.7916 57.2008) (end 59.7408 57.2008) (width 0.25) (layer "F.Cu") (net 5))
 (segment (start 68.472931 59.517669) (end 70.402331 59.517669) (width 0.25) (layer "F.Cu") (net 5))
 (segment (start 68.472931 59.517669) (end 68.4906 59.5) (width 0.25) (layer "F.Cu") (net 5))
 (segment (start 70.402331 59.517669) (end 70.42 59.5) (width 0.25) (layer "F.Cu") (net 5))
 (segment (start 59.7408 57.2008) (end 56.4416 60.5) (width 0.25) (layer "F.Cu") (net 5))
 (segment (start 56.4416 60.5) (end 54.98 60.5) (width 0.25) (layer "F.Cu") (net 5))
 (segment (start 68.472931 59.517669) (end 68.455262 59.5) (width 0.25) (layer "F.Cu") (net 5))
 (segment (start 70.352331 59.517669) (end 70.37 59.5) (width 0.25) (layer "F.Cu") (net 5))
 (via (at 59.7916 57.2008) (size 0.6) (drill 0.3) (layers "F.Cu" "B.Cu") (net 5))
 (via (at 68.472931 59.517669) (size 0.6) (drill 0.3) (layers "F.Cu" "B.Cu") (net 5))
 (segment (start 61.4492 57.2008) (end 59.7916 57.2008) (width 0.25) (layer "B.Cu") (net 5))
 (segment (start 68.472931 59.517669) (end 65.791469 59.517669) (width 0.25) (layer "B.Cu") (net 5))
 (segment (start 65.791469 59.517669) (end 63.4638 57.19) (width 0.25) (layer "B.Cu") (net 5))
 (segment (start 61.46 57.19) (end 61.4492 57.2008) (width 0.25) (layer "B.Cu") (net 5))
 (segment (start 63.4638 57.19) (end 61.46 57.19) (width 0.25) (layer "B.Cu") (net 5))
 (segment (start 63.627 54.4068) (end 63.1698 54.864) (width 0.25) (layer "F.Cu") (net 9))
 (segment (start 64.5202 65.881) (end 64.5202 66.081) (width 0.25) (layer "F.Cu") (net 9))
 (segment (start 62.8402 65.941) (end 62.8452 65.936) (width 0.25) (layer "F.Cu") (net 9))
 (segment (start 63.5452 65.936) (end 64.4652 65.936) (width 0.25) (layer "F.Cu") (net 9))
 (segment (start 61.6202 65.941) (end 60.4038 65.941) (width 0.25) (layer "F.Cu") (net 9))
 (segment (start 65.6082 68.5546) (end 65.1502 68.0966) (width 0.25) (layer "F.Cu") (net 9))
 (segment (start 58.55 65.1) (end 58.55 65.5858) (width 0.25) (layer "F.Cu") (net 9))
 (segment (start 62.8452 65.936) (end 63.5452 65.936) (width 0.25) (layer "F.Cu") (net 9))
 (segment (start 61.727 52.847) (end 62.1942 52.847) (width 0.25) (layer "F.Cu") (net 9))
 (segment (start 68.5546 68.5292) (end 65.6336 68.5292) (width 0.25) (layer "F.Cu") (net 9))
 (segment (start 65.1502 66.711) (end 65.1502 67.481) (width 0.25) (layer "F.Cu") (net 9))
 (segment (start 68.4754 54.6354) (end 68.83 54.99) (width 0.25) (layer "F.Cu") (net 9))
 (segment (start 63.627 53.497) (end 64.1396 53.497) (width 0.25) (layer "F.Cu") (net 9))
 (segment (start 65.278 54.6354) (end 68.4754 54.6354) (width 0.25) (layer "F.Cu") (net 9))
 (segment (start 62.1942 52.847) (end 62.8442 53.497) (width 0.25) (layer "F.Cu") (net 9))
 (segment (start 64.5202 66.081) (end 65.1502 66.711) (width 0.25) (layer "F.Cu") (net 9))
 (segment (start 61.6202 65.941) (end 62.8402 65.941) (width 0.25) (layer "F.Cu") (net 9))
 (segment (start 59.5628 65.1) (end 58.55 65.1) (width 0.25) (layer "F.Cu") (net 9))
 (segment (start 65.6336 68.5292) (end 65.6082 68.5546) (width 0.25) (layer "F.Cu") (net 9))
 (segment (start 63.627 53.497) (end 63.627 54.4068) (width 0.25) (layer "F.Cu") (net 9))
 (segment (start 64.1396 53.497) (end 65.278 54.6354) (width 0.25) (layer "F.Cu") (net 9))
 (segment (start 69.9008 67.183) (end 68.5546 68.5292) (width 0.25) (layer "F.Cu") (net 9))
 (segment (start 60.4038 65.941) (end 59.5628 65.1) (width 0.25) (layer "F.Cu") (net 9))
 (segment (start 69.9008 63.881) (end 69.9008 67.183) (width 0.25) (layer "F.Cu") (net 9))
 (segment (start 62.8442 53.497) (end 63.627 53.497) (width 0.25) (layer "F.Cu") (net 9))
 (segment (start 65.1502 68.0966) (end 65.1502 67.481) (width 0.25) (layer "F.Cu") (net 9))
 (segment (start 64.4652 65.936) (end 64.5202 65.881) (width 0.25) (layer "F.Cu") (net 9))
 (via (at 69.9008 63.881) (size 0.6) (drill 0.3) (layers "F.Cu" "B.Cu") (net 9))
 (via (at 68.83 54.99) (size 0.6) (drill 0.3) (layers "F.Cu" "B.Cu") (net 9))
 (segment (start 69.9008 56.0832) (end 68.83 55.0124) (width 0.25) (layer "B.Cu") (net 9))
 (segment (start 68.83 55.0124) (end 68.83 54.99) (width 0.25) (layer "B.Cu") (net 9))
 (segment (start 69.9008 63.881) (end 69.9008 56.0832) (width 0.25) (layer "B.Cu") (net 9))
 (segment (start 68.426 63.981) (end 68.4276 63.9826) (width 0.25) (layer "F.Cu") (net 1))
 (segment (start 66.802 61.9252) (end 66.802 63.3476) (width 0.25) (layer "F.Cu") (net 1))
 (segment (start 62.7 59.2125) (end 64.0893 59.2125) (width 0.25) (layer "F.Cu") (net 1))
 (segment (start 66.7952 63.981) (end 68.426 63.981) (width 0.25) (layer "F.Cu") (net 1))
 (segment (start 64.0893 59.2125) (end 66.802 61.9252) (width 0.25) (layer "F.Cu") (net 1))
 (segment (start 66.7952 63.3544) (end 66.7952 63.981) (width 0.25) (layer "F.Cu") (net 1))
 (segment (start 66.802 63.3476) (end 66.7952 63.3544) (width 0.25) (layer "F.Cu") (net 1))
 (segment (start 60.0375 60.7875) (end 62.7 60.7875) (width 0.25) (layer "F.Cu") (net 2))
 (segment (start 57.6 63.225) (end 57.6 62.56) (width 0.25) (layer "F.Cu") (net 2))
 (segment (start 57.6 63.225) (end 60.0375 60.7875) (width 0.25) (layer "F.Cu") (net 2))
 (segment (start 62.0058 63.225) (end 59.5 63.225) (width 0.25) (layer "F.Cu") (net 8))
 (segment (start 59.545 63.18) (end 59.5 63.225) (width 0.25) (layer "F.Cu") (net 8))
 (segment (start 64.5202 63.981) (end 62.7618 63.981) (width 0.25) (layer "F.Cu") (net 8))
 (segment (start 62.7618 63.981) (end 62.0058 63.225) (width 0.25) (layer "F.Cu") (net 8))
 (segment (start 66.7952 67.346) (end 66.6602 67.481) (width 0.25) (layer "F.Cu") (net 7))
 (segment (start 67.7164 67.3608) (end 68.4276 67.3608) (width 0.25) (layer "F.Cu") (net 7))
 (segment (start 66.7952 65.881) (end 66.7952 67.196) (width 0.25) (layer "F.Cu") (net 7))
 (segment (start 66.5226 67.481) (end 67.5962 67.481) (width 0.25) (layer "F.Cu") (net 7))
 (segment (start 66.5226 67.481) (end 66.1702 67.481) (width 0.25) (layer "F.Cu") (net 7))
 (segment (start 66.7952 67.196) (end 66.7952 67.346) (width 0.25) (layer "F.Cu") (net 7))
 (segment (start 66.6602 67.481) (end 66.5226 67.481) (width 0.25) (layer "F.Cu") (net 7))
 (segment (start 67.5962 67.481) (end 67.7164 67.3608) (width 0.25) (layer "F.Cu") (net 7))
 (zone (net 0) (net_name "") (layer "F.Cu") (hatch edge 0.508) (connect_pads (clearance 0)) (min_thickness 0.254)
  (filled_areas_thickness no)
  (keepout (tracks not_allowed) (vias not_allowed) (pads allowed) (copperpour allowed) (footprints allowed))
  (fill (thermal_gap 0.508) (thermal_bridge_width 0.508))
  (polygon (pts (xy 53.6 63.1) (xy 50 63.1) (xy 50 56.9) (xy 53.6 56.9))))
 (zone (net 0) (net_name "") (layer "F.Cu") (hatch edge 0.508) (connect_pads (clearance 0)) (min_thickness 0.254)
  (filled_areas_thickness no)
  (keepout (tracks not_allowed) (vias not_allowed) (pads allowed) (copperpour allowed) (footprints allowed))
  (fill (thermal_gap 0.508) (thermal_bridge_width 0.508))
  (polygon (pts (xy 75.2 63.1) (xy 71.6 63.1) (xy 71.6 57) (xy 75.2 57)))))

